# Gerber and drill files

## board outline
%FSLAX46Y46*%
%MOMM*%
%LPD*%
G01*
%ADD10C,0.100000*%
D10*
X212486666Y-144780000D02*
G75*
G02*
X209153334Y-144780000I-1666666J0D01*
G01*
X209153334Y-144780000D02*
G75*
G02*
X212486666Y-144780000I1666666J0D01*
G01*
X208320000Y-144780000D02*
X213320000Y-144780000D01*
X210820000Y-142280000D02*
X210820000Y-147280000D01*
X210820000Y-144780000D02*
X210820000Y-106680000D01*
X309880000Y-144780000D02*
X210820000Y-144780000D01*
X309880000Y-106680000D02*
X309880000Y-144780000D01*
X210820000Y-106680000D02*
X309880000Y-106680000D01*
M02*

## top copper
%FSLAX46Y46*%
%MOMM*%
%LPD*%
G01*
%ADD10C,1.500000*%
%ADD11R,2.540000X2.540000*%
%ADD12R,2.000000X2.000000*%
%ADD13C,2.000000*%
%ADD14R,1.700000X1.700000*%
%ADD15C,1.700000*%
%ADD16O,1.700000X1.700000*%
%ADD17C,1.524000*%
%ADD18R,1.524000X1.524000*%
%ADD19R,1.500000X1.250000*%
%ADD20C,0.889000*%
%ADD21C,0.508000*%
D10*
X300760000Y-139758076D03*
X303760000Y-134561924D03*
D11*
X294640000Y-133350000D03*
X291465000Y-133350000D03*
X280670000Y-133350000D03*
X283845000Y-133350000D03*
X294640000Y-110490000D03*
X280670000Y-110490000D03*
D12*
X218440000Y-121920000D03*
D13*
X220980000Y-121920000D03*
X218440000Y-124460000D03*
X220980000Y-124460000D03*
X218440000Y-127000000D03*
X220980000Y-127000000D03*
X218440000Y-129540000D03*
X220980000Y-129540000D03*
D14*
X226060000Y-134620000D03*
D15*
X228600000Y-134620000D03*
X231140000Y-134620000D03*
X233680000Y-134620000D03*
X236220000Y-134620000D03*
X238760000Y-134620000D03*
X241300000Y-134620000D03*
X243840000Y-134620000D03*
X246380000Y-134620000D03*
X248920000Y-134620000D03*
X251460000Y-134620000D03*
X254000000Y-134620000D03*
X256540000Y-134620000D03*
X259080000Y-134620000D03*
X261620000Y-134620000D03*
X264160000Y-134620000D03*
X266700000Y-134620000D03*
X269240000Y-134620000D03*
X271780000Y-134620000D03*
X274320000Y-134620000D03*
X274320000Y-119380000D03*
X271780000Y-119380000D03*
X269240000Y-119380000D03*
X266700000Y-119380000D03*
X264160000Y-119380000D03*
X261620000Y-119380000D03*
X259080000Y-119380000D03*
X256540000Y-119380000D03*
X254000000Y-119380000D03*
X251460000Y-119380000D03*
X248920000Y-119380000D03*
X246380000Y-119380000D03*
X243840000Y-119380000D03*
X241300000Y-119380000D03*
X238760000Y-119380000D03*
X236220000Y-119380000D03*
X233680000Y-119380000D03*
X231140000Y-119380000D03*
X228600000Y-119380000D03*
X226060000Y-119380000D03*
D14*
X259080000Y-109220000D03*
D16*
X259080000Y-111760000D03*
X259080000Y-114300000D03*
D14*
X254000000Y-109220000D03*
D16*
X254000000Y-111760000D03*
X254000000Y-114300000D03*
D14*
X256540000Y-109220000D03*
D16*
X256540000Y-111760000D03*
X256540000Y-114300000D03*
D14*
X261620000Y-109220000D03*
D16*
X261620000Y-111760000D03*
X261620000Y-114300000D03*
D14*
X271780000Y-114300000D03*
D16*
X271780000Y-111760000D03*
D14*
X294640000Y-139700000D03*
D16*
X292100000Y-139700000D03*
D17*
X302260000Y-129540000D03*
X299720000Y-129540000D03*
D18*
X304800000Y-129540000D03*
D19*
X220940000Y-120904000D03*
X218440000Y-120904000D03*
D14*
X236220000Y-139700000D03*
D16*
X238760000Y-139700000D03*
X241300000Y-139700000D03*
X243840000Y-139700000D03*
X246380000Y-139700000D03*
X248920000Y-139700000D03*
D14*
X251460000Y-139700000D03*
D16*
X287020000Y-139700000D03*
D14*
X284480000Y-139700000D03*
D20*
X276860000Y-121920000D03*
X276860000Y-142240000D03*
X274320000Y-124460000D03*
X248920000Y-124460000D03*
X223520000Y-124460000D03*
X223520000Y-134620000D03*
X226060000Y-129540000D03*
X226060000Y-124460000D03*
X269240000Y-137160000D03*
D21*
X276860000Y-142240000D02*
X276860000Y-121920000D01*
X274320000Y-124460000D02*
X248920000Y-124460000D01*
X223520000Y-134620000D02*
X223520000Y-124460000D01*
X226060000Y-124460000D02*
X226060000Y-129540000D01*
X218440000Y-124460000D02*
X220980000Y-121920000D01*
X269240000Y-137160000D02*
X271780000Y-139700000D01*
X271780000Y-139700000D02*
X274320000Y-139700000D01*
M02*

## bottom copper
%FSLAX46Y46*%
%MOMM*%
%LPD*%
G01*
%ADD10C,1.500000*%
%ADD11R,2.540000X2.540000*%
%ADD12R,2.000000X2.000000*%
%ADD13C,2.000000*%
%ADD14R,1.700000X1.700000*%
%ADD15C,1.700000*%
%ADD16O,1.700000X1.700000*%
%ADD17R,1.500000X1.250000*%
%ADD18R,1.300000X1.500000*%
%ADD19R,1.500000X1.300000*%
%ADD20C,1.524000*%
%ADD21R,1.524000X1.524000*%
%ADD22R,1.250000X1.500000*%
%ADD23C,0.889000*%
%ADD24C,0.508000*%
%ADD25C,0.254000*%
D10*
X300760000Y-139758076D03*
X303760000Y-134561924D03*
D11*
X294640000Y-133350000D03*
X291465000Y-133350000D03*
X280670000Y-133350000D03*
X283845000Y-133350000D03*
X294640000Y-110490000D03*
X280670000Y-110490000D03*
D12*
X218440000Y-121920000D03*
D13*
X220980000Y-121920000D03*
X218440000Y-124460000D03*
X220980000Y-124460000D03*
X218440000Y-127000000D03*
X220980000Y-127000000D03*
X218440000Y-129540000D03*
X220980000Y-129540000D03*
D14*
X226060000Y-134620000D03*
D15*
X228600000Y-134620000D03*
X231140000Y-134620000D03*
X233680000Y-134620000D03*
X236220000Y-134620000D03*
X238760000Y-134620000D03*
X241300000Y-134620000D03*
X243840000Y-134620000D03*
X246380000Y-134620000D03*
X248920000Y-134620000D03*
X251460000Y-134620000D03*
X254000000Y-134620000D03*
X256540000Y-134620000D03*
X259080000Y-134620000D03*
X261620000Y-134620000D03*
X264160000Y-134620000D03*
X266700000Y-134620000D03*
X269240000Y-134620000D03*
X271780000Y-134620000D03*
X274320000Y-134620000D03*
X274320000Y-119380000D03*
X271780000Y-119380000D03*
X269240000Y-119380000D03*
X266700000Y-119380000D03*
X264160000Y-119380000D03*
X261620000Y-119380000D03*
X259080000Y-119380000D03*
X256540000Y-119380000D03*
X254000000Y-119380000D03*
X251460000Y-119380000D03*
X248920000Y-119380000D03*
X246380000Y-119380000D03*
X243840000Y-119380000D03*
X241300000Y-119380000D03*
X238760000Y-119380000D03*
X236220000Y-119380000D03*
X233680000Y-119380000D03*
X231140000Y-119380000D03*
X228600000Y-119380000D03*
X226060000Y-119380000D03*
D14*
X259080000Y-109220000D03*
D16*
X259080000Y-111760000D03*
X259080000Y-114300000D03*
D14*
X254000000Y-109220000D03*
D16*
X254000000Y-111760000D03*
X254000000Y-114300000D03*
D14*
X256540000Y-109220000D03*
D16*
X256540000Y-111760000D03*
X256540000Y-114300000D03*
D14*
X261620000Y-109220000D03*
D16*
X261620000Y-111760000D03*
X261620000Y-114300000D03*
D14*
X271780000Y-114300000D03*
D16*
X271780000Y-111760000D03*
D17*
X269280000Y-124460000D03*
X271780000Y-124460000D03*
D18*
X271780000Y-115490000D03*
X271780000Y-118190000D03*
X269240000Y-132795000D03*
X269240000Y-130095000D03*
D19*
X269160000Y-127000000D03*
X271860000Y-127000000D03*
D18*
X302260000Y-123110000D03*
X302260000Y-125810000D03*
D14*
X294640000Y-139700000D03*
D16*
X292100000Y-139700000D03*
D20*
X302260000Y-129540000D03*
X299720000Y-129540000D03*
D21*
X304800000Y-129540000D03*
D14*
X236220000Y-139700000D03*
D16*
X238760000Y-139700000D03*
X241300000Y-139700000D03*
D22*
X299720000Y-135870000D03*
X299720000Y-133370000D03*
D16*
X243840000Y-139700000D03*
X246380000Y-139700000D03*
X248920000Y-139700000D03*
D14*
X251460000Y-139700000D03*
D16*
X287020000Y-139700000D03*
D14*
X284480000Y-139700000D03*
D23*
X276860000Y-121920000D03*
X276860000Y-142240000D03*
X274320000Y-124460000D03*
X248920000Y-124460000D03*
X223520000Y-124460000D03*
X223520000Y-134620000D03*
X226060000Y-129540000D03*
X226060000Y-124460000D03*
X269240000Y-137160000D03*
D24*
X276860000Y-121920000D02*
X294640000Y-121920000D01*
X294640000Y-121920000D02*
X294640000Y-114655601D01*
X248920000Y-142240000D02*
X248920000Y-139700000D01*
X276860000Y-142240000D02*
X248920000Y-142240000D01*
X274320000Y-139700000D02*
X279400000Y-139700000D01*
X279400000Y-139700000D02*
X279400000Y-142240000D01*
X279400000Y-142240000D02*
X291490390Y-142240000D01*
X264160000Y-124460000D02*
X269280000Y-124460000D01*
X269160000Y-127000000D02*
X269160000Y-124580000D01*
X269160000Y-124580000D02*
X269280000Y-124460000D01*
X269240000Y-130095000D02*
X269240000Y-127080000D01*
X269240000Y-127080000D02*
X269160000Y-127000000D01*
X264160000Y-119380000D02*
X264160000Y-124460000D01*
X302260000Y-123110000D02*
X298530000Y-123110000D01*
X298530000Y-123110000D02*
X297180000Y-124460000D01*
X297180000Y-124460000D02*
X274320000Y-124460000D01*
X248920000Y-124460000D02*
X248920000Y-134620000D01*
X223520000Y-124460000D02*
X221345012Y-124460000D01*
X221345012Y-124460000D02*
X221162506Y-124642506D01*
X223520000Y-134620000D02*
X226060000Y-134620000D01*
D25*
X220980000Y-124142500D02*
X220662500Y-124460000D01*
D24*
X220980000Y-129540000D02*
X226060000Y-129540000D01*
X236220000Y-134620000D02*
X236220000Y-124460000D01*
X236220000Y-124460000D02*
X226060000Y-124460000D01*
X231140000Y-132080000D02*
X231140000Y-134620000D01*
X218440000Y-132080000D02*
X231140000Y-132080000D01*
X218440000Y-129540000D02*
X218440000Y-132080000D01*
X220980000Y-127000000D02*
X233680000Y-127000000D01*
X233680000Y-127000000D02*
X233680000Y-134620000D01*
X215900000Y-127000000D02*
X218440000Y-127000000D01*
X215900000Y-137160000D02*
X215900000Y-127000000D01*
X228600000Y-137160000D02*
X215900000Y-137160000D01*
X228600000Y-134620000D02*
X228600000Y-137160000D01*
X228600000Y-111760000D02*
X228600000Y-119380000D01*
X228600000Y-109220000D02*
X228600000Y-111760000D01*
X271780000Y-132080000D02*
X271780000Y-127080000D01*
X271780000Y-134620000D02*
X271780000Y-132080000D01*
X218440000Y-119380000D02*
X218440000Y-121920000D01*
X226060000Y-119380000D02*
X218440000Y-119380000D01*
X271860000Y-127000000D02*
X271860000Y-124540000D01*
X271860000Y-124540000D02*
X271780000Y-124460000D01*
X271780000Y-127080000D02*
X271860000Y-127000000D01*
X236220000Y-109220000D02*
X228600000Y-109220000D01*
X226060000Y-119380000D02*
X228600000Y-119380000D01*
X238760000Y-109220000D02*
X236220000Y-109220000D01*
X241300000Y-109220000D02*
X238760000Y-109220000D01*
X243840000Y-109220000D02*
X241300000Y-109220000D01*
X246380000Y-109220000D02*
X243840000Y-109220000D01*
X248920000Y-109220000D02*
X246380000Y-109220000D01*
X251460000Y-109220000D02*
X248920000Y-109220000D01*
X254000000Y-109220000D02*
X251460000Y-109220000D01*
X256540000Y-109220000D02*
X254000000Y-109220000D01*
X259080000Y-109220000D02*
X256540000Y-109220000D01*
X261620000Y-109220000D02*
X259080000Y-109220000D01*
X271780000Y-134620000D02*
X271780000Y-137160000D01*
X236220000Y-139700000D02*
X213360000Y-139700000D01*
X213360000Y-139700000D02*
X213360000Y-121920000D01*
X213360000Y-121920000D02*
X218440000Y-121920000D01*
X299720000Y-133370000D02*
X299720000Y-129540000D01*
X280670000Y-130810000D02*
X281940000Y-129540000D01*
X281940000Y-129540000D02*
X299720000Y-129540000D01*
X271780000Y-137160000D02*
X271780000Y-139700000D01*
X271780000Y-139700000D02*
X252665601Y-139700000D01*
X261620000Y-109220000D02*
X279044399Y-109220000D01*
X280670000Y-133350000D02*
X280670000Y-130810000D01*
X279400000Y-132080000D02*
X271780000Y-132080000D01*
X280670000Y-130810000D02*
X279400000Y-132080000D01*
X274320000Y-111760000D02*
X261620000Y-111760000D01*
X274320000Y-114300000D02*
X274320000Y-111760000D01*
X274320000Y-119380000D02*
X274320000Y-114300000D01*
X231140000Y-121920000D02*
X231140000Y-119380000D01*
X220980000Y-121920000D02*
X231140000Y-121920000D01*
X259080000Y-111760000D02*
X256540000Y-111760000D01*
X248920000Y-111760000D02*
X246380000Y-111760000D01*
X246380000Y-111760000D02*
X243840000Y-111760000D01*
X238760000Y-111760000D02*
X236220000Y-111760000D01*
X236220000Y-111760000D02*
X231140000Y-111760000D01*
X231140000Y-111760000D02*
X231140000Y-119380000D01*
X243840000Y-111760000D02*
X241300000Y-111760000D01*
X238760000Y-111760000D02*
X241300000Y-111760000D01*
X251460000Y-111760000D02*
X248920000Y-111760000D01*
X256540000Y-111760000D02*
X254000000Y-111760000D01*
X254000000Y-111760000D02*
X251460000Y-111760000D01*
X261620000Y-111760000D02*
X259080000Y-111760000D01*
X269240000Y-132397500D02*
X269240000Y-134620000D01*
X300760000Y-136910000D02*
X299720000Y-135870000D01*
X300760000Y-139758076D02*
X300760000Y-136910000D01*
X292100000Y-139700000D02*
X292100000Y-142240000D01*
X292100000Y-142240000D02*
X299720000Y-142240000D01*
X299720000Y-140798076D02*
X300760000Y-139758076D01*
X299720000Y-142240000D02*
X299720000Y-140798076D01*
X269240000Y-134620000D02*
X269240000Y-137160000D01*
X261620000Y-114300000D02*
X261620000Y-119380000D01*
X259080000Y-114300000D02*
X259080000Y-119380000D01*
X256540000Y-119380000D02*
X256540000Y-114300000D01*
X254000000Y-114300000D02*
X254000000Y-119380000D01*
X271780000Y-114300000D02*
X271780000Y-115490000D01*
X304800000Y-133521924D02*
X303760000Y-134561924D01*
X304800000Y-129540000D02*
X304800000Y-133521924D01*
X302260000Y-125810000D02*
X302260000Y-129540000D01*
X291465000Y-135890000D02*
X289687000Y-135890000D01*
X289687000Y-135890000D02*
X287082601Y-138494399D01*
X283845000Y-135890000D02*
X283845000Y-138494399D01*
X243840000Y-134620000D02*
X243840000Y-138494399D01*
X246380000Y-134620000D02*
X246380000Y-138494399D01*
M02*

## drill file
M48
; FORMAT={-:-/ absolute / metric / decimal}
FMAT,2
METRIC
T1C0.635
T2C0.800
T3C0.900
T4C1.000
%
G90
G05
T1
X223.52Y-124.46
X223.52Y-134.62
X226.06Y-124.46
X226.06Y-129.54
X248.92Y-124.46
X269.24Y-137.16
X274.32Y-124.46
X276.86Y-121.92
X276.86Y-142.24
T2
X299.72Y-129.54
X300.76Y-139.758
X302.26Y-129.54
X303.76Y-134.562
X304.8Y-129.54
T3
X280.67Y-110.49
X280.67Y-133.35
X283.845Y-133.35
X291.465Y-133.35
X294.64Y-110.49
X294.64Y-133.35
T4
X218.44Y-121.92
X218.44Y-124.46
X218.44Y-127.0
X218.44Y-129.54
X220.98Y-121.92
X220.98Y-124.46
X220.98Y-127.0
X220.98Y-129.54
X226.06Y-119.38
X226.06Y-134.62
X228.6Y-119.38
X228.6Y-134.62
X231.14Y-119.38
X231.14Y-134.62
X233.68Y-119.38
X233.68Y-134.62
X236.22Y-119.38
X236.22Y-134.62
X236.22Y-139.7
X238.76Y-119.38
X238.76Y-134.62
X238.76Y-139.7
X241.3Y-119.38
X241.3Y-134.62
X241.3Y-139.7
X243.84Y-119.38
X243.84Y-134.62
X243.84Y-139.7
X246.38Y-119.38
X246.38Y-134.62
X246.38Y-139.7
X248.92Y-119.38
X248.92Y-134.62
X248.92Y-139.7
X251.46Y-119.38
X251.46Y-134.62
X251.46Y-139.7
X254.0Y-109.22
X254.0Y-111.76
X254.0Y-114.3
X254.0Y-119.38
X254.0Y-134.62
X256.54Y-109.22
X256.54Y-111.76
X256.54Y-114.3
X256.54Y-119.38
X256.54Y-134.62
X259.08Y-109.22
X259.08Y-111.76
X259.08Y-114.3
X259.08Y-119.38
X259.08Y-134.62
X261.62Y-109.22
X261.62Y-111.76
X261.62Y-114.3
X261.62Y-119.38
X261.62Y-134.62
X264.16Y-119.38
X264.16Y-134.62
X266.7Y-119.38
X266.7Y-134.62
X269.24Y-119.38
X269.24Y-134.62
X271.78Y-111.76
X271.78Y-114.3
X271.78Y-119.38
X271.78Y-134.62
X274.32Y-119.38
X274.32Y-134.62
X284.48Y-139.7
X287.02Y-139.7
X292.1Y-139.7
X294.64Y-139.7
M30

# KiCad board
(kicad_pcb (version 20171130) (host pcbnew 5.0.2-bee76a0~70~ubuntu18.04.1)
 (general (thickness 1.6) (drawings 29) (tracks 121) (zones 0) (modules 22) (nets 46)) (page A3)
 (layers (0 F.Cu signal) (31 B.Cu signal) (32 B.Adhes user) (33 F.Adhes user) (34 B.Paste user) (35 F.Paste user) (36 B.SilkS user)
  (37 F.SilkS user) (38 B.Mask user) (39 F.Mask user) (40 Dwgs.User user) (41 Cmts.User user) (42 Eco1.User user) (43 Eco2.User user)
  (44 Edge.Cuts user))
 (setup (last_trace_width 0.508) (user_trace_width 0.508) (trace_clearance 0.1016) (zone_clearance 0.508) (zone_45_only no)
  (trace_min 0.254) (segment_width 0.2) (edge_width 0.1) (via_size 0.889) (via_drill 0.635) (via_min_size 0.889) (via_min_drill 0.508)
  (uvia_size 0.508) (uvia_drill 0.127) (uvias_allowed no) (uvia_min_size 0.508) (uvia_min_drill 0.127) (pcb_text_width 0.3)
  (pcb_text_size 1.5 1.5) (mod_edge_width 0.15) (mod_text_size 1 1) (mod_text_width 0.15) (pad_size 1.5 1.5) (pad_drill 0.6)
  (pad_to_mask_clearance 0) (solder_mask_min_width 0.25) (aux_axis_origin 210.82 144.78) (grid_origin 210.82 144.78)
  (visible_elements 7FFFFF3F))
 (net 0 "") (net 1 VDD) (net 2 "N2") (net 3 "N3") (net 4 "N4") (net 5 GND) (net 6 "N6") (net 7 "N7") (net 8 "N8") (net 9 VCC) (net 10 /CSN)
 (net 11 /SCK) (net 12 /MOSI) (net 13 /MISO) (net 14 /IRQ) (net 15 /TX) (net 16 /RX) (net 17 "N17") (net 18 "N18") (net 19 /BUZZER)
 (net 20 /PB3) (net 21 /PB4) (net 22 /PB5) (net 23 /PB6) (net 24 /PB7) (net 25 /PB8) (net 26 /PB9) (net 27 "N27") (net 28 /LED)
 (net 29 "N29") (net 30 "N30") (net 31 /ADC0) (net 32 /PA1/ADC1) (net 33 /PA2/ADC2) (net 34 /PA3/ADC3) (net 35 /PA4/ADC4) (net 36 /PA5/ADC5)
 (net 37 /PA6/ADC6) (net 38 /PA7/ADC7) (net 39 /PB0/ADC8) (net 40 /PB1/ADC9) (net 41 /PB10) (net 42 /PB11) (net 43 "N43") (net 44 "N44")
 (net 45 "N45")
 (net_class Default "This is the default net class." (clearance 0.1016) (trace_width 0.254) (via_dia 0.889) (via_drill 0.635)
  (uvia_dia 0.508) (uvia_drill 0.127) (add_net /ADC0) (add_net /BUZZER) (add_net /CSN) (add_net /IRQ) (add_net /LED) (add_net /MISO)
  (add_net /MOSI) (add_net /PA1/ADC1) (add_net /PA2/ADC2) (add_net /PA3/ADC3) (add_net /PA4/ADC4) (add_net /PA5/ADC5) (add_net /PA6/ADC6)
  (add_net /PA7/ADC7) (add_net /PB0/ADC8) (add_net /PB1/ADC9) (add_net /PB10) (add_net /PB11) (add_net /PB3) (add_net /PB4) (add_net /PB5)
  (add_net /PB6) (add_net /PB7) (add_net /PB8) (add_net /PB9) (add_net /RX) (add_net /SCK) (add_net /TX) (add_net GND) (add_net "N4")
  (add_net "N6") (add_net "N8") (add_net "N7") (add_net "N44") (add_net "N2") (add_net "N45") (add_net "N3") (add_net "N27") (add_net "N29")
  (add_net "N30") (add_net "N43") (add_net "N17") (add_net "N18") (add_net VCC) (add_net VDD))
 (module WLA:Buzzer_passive (layer F.Cu) (at 302.26 137.16 60)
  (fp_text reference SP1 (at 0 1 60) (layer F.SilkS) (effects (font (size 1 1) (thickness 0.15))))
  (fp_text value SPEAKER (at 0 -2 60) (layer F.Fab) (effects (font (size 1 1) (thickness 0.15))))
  (pad 1 thru_hole circle (at -3 0 60) (size 1.5 1.5) (drill 0.8) (layers *.Cu *.Mask) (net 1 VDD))
  (pad 2 thru_hole circle (at 3 0 60) (size 1.5 1.5) (drill 0.8) (layers *.Cu *.Mask) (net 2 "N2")))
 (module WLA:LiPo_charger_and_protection (layer F.Cu) (at 287.655 121.92 270)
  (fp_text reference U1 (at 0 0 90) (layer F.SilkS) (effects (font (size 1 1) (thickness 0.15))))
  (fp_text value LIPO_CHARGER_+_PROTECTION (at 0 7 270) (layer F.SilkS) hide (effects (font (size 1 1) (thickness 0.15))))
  (pad 3 thru_hole rect (at 11.43 -6.985 270) (size 2.54 2.54) (drill 0.9) (layers *.Cu *.Mask F.SilkS) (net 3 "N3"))
  (pad 1 thru_hole rect (at 11.43 -3.81 270) (size 2.54 2.54) (drill 0.9) (layers *.Cu *.Mask F.SilkS) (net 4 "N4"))
  (pad 4 thru_hole rect (at 11.43 6.985 270) (size 2.54 2.54) (drill 0.9) (layers *.Cu *.Mask F.SilkS) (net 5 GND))
  (pad 2 thru_hole rect (at 11.43 3.81 270) (size 2.54 2.54) (drill 0.9) (layers *.Cu *.Mask F.SilkS) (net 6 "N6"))
  (pad 5 thru_hole rect (at -11.43 -6.985 270) (size 2.54 2.54) (drill 0.9) (layers *.Cu *.Mask F.SilkS) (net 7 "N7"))
  (pad 6 thru_hole rect (at -11.43 6.985 270) (size 2.54 2.54) (drill 0.9) (layers *.Cu *.Mask F.SilkS) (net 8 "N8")))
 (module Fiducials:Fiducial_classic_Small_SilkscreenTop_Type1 (layer F.Cu) (at 210.82 144.78)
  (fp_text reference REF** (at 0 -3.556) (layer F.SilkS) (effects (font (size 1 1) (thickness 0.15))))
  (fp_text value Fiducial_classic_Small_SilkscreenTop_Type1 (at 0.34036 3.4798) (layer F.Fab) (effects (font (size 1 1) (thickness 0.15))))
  (pad ~ smd circle (at 0 0) (size 4.50088 4.50088) (layers F.Mask) (solder_mask_margin 2.99974)))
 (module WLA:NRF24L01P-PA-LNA (layer F.Cu) (at 218.44 125.73 270)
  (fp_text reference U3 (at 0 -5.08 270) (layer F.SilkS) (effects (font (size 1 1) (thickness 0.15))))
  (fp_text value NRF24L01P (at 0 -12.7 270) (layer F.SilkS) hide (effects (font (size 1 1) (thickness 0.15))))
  (pad 1 thru_hole rect (at -3.81 0 270) (size 2 2) (drill 1) (layers *.Cu *.Mask F.SilkS) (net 5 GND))
  (pad 2 thru_hole circle (at -3.81 -2.54 270) (size 2 2) (drill 1) (layers *.Cu *.Mask F.SilkS) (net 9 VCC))
  (pad 3 thru_hole circle (at -1.27 0 270) (size 2 2) (drill 1) (layers *.Cu *.Mask F.SilkS) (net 9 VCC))
  (pad 4 thru_hole circle (at -1.27 -2.54 270) (size 2 2) (drill 1) (layers *.Cu *.Mask F.SilkS) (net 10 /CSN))
  (pad 5 thru_hole circle (at 1.27 0 270) (size 2 2) (drill 1) (layers *.Cu *.Mask F.SilkS) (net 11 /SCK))
  (pad 6 thru_hole circle (at 1.27 -2.54 270) (size 2 2) (drill 1) (layers *.Cu *.Mask F.SilkS) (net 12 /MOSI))
  (pad 7 thru_hole circle (at 3.81 0 270) (size 2 2) (drill 1) (layers *.Cu *.Mask F.SilkS) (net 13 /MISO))
  (pad 8 thru_hole circle (at 3.81 -2.54 270) (size 2 2) (drill 1) (layers *.Cu *.Mask F.SilkS) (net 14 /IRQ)))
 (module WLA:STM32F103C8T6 (layer F.Cu) (at 250.19 127)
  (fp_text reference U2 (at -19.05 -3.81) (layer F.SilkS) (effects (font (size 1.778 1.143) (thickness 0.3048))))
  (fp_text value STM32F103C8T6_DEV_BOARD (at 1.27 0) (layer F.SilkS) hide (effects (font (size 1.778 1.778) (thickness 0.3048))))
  (pad 1 thru_hole rect (at -24.13 7.62) (size 1.7 1.7) (drill 1) (layers *.Cu *.Mask F.SilkS) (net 10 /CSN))
  (pad 2 thru_hole circle (at -21.59 7.62) (size 1.7 1.7) (drill 1) (layers *.Cu *.Mask F.SilkS) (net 11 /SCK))
  (pad 3 thru_hole circle (at -19.05 7.62) (size 1.7 1.7) (drill 1) (layers *.Cu *.Mask F.SilkS) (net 13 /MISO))
  (pad 4 thru_hole circle (at -16.51 7.62) (size 1.7 1.7) (drill 1) (layers *.Cu *.Mask F.SilkS) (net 12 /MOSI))
  (pad 5 thru_hole circle (at -13.97 7.62) (size 1.7 1.7) (drill 1) (layers *.Cu *.Mask F.SilkS) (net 14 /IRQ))
  (pad 6 thru_hole circle (at -11.43 7.62) (size 1.7 1.7) (drill 1) (layers *.Cu *.Mask F.SilkS) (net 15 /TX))
  (pad 7 thru_hole circle (at -8.89 7.62) (size 1.7 1.7) (drill 1) (layers *.Cu *.Mask F.SilkS) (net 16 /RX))
  (pad 8 thru_hole circle (at -6.35 7.62) (size 1.7 1.7) (drill 1) (layers *.Cu *.Mask F.SilkS) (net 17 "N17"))
  (pad 9 thru_hole circle (at -3.81 7.62) (size 1.7 1.7) (drill 1) (layers *.Cu *.Mask F.SilkS) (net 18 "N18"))
  (pad 10 thru_hole circle (at -1.27 7.62) (size 1.7 1.7) (drill 1) (layers *.Cu *.Mask F.SilkS) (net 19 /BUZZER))
  (pad 11 thru_hole circle (at 1.27 7.62) (size 1.7 1.7) (drill 1) (layers *.Cu *.Mask F.SilkS) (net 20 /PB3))
  (pad 12 thru_hole circle (at 3.81 7.62) (size 1.7 1.7) (drill 1) (layers *.Cu *.Mask F.SilkS) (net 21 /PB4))
  (pad 13 thru_hole circle (at 6.35 7.62) (size 1.7 1.7) (drill 1) (layers *.Cu *.Mask F.SilkS) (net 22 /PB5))
  (pad 14 thru_hole circle (at 8.89 7.62) (size 1.7 1.7) (drill 1) (layers *.Cu *.Mask F.SilkS) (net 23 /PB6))
  (pad 15 thru_hole circle (at 11.43 7.62) (size 1.7 1.7) (drill 1) (layers *.Cu *.Mask F.SilkS) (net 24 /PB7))
  (pad 16 thru_hole circle (at 13.97 7.62) (size 1.7 1.7) (drill 1) (layers *.Cu *.Mask F.SilkS) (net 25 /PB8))
  (pad 17 thru_hole circle (at 16.51 7.62) (size 1.7 1.7) (drill 1) (layers *.Cu *.Mask F.SilkS) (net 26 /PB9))
  (pad 18 thru_hole circle (at 19.05 7.62) (size 1.7 1.7) (drill 1) (layers *.Cu *.Mask F.SilkS) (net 1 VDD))
  (pad 19 thru_hole circle (at 21.59 7.62) (size 1.7 1.7) (drill 1) (layers *.Cu *.Mask F.SilkS) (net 5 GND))
  (pad 20 thru_hole circle (at 24.13 7.62) (size 1.7 1.7) (drill 1) (layers *.Cu *.Mask F.SilkS) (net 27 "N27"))
  (pad 21 thru_hole circle (at 24.13 -7.62) (size 1.7 1.7) (drill 1) (layers *.Cu *.Mask F.SilkS) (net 9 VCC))
  (pad 22 thru_hole circle (at 21.59 -7.62) (size 1.7 1.7) (drill 1) (layers *.Cu *.Mask F.SilkS) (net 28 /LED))
  (pad 23 thru_hole circle (at 19.05 -7.62) (size 1.7 1.7) (drill 1) (layers *.Cu *.Mask F.SilkS) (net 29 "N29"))
  (pad 24 thru_hole circle (at 16.51 -7.62) (size 1.7 1.7) (drill 1) (layers *.Cu *.Mask F.SilkS) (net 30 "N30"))
  (pad 25 thru_hole circle (at 13.97 -7.62) (size 1.7 1.7) (drill 1) (layers *.Cu *.Mask F.SilkS) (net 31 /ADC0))
  (pad 26 thru_hole circle (at 11.43 -7.62) (size 1.7 1.7) (drill 1) (layers *.Cu *.Mask F.SilkS) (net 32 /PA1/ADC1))
  (pad 27 thru_hole circle (at 8.89 -7.62) (size 1.7 1.7) (drill 1) (layers *.Cu *.Mask F.SilkS) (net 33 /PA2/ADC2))
  (pad 28 thru_hole circle (at 6.35 -7.62) (size 1.7 1.7) (drill 1) (layers *.Cu *.Mask F.SilkS) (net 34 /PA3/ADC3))
  (pad 29 thru_hole circle (at 3.81 -7.62) (size 1.7 1.7) (drill 1) (layers *.Cu *.Mask F.SilkS) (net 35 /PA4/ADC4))
  (pad 30 thru_hole circle (at 1.27 -7.62) (size 1.7 1.7) (drill 1) (layers *.Cu *.Mask F.SilkS) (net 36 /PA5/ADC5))
  (pad 31 thru_hole circle (at -1.27 -7.62) (size 1.7 1.7) (drill 1) (layers *.Cu *.Mask F.SilkS) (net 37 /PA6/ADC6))
  (pad 32 thru_hole circle (at -3.81 -7.62) (size 1.7 1.7) (drill 1) (layers *.Cu *.Mask F.SilkS) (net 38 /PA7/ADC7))
  (pad 33 thru_hole circle (at -6.35 -7.62) (size 1.7 1.7) (drill 1) (layers *.Cu *.Mask F.SilkS) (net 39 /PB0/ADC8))
  (pad 34 thru_hole circle (at -8.89 -7.62) (size 1.7 1.7) (drill 1) (layers *.Cu *.Mask F.SilkS) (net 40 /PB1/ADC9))
  (pad 35 thru_hole circle (at -11.43 -7.62) (size 1.7 1.7) (drill 1) (layers *.Cu *.Mask F.SilkS) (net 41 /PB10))
  (pad 36 thru_hole circle (at -13.97 -7.62) (size 1.7 1.7) (drill 1) (layers *.Cu *.Mask F.SilkS) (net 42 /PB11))
  (pad 37 thru_hole circle (at -16.51 -7.62) (size 1.7 1.7) (drill 1) (layers *.Cu *.Mask F.SilkS) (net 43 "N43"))
  (pad 38 thru_hole circle (at -19.05 -7.62) (size 1.7 1.7) (drill 1) (layers *.Cu *.Mask F.SilkS) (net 9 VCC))
  (pad 39 thru_hole circle (at -21.59 -7.62) (size 1.7 1.7) (drill 1) (layers *.Cu *.Mask F.SilkS) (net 5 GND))
  (pad 40 thru_hole circle (at -24.13 -7.62) (size 1.7 1.7) (drill 1) (layers *.Cu *.Mask F.SilkS) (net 5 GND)))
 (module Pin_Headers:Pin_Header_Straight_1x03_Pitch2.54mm (layer F.Cu) (at 259.08 109.22)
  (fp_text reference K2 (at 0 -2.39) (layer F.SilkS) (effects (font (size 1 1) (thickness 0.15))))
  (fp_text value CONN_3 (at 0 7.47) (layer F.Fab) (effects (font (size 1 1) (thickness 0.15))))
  (pad 1 thru_hole rect (at 0 0) (size 1.7 1.7) (drill 1) (layers *.Cu *.Mask) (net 5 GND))
  (pad 2 thru_hole oval (at 0 2.54) (size 1.7 1.7) (drill 1) (layers *.Cu *.Mask) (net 9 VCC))
  (pad 3 thru_hole oval (at 0 5.08) (size 1.7 1.7) (drill 1) (layers *.Cu *.Mask) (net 33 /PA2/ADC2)))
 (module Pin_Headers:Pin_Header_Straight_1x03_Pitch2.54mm (layer F.Cu) (at 254 109.22)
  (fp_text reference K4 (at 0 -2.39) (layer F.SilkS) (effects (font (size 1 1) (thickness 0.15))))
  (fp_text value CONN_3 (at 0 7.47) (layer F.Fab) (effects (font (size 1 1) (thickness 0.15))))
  (pad 1 thru_hole rect (at 0 0) (size 1.7 1.7) (drill 1) (layers *.Cu *.Mask) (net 5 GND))
  (pad 2 thru_hole oval (at 0 2.54) (size 1.7 1.7) (drill 1) (layers *.Cu *.Mask) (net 9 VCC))
  (pad 3 thru_hole oval (at 0 5.08) (size 1.7 1.7) (drill 1) (layers *.Cu *.Mask) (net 35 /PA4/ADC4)))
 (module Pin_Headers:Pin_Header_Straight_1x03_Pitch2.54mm (layer F.Cu) (at 256.54 109.22)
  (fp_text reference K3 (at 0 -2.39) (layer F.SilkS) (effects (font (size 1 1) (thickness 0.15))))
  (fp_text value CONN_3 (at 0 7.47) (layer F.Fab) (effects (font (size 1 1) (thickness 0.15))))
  (pad 1 thru_hole rect (at 0 0) (size 1.7 1.7) (drill 1) (layers *.Cu *.Mask) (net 5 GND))
  (pad 2 thru_hole oval (at 0 2.54) (size 1.7 1.7) (drill 1) (layers *.Cu *.Mask) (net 9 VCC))
  (pad 3 thru_hole oval (at 0 5.08) (size 1.7 1.7) (drill 1) (layers *.Cu *.Mask) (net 34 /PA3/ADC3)))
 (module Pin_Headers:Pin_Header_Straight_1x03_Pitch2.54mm (layer F.Cu) (at 261.62 109.22)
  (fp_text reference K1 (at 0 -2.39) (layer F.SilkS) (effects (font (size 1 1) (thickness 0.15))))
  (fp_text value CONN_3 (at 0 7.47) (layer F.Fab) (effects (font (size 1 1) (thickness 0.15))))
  (pad 1 thru_hole rect (at 0 0) (size 1.7 1.7) (drill 1) (layers *.Cu *.Mask) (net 5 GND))
  (pad 2 thru_hole oval (at 0 2.54) (size 1.7 1.7) (drill 1) (layers *.Cu *.Mask) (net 9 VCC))
  (pad 3 thru_hole oval (at 0 5.08) (size 1.7 1.7) (drill 1) (layers *.Cu *.Mask) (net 32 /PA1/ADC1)))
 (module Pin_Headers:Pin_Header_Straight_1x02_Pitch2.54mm (layer F.Cu) (at 271.78 114.3 180)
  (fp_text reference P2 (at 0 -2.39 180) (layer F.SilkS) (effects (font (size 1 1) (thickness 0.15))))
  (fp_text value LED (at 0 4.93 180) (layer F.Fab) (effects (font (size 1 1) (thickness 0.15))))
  (pad 1 thru_hole rect (at 0 0 180) (size 1.7 1.7) (drill 1) (layers *.Cu *.Mask) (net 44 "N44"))
  (pad 2 thru_hole oval (at 0 2.54 180) (size 1.7 1.7) (drill 1) (layers *.Cu *.Mask) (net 9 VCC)))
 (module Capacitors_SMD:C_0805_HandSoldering (layer B.Cu) (at 270.53 124.46)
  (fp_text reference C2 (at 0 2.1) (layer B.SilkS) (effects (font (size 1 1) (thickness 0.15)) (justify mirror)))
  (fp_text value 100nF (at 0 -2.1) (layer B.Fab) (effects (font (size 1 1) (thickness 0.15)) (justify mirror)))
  (pad 1 smd rect (at -1.25 0) (size 1.5 1.25) (layers B.Cu B.Paste B.Mask) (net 31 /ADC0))
  (pad 2 smd rect (at 1.25 0) (size 1.5 1.25) (layers B.Cu B.Paste B.Mask) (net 5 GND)))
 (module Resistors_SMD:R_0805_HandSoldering (layer B.Cu) (at 271.78 116.84 270)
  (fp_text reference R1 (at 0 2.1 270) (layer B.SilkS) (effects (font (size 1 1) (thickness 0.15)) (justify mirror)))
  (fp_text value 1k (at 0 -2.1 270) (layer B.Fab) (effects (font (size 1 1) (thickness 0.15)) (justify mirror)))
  (pad 1 smd rect (at -1.35 0 270) (size 1.5 1.3) (layers B.Cu B.Paste B.Mask) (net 44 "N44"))
  (pad 2 smd rect (at 1.35 0 270) (size 1.5 1.3) (layers B.Cu B.Paste B.Mask) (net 28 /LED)))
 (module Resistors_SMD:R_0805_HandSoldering (layer B.Cu) (at 269.24 131.445 90)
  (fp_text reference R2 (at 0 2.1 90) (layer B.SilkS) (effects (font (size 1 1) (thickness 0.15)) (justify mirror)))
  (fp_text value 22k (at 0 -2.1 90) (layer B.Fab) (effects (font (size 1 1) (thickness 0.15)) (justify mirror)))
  (pad 1 smd rect (at -1.35 0 90) (size 1.5 1.3) (layers B.Cu B.Paste B.Mask) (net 1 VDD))
  (pad 2 smd rect (at 1.35 0 90) (size 1.5 1.3) (layers B.Cu B.Paste B.Mask) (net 31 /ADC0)))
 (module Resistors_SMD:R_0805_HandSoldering (layer B.Cu) (at 270.51 127)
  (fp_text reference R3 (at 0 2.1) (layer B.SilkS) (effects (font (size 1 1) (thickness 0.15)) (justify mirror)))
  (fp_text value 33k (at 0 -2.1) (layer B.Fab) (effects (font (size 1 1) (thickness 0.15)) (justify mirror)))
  (pad 1 smd rect (at -1.35 0) (size 1.5 1.3) (layers B.Cu B.Paste B.Mask) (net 31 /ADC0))
  (pad 2 smd rect (at 1.35 0) (size 1.5 1.3) (layers B.Cu B.Paste B.Mask) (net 5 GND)))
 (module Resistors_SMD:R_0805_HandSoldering (layer B.Cu) (at 302.26 124.46 270)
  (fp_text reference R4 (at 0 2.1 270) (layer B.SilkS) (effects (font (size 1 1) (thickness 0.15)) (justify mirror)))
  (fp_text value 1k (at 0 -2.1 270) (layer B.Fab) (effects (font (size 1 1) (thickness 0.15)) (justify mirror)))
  (pad 1 smd rect (at -1.35 0 270) (size 1.5 1.3) (layers B.Cu B.Paste B.Mask) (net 19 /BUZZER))
  (pad 2 smd rect (at 1.35 0 270) (size 1.5 1.3) (layers B.Cu B.Paste B.Mask) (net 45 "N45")))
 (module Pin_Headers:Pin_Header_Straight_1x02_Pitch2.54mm (layer F.Cu) (at 294.64 139.7 270)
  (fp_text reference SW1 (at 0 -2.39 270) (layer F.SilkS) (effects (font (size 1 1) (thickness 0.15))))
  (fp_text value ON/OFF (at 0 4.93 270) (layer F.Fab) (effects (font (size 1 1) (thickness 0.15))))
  (pad 1 thru_hole rect (at 0 0 270) (size 1.7 1.7) (drill 1) (layers *.Cu *.Mask) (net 3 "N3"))
  (pad 2 thru_hole oval (at 0 2.54 270) (size 1.7 1.7) (drill 1) (layers *.Cu *.Mask) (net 1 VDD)))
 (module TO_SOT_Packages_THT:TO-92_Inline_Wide (layer F.Cu) (at 304.8 129.54 180)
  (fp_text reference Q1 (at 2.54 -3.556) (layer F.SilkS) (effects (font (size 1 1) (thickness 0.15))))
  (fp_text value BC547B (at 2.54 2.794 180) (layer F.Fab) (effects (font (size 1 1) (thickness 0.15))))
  (pad 2 thru_hole circle (at 2.54 0 270) (size 1.524 1.524) (drill 0.8) (layers *.Cu *.Mask) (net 45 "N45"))
  (pad 3 thru_hole circle (at 5.08 0 270) (size 1.524 1.524) (drill 0.8) (layers *.Cu *.Mask) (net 5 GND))
  (pad 1 thru_hole rect (at 0 0 270) (size 1.524 1.524) (drill 0.8) (layers *.Cu *.Mask) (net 2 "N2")))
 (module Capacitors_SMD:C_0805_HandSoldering (layer F.Cu) (at 219.69 120.904 180)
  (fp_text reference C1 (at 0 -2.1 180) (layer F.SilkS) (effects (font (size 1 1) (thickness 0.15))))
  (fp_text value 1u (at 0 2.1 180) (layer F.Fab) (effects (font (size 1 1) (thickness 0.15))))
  (pad 1 smd rect (at -1.25 0 180) (size 1.5 1.25) (layers F.Cu F.Paste F.Mask) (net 9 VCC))
  (pad 2 smd rect (at 1.25 0 180) (size 1.5 1.25) (layers F.Cu F.Paste F.Mask) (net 5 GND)))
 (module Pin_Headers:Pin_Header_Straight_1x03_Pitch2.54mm (layer F.Cu) (at 236.22 139.7 90)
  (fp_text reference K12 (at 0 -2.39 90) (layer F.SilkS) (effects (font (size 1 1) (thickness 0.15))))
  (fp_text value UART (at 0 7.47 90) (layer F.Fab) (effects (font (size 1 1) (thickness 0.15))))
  (pad 1 thru_hole rect (at 0 0 90) (size 1.7 1.7) (drill 1) (layers *.Cu *.Mask) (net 5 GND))
  (pad 2 thru_hole oval (at 0 2.54 90) (size 1.7 1.7) (drill 1) (layers *.Cu *.Mask) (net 16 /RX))
  (pad 3 thru_hole oval (at 0 5.08 90) (size 1.7 1.7) (drill 1) (layers *.Cu *.Mask) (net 15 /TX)))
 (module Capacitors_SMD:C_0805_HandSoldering (layer B.Cu) (at 299.72 134.62 90)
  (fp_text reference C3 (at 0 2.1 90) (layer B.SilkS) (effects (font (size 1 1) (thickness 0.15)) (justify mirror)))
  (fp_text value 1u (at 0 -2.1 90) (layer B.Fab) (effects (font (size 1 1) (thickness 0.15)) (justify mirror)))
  (pad 1 smd rect (at -1.25 0 90) (size 1.5 1.25) (layers B.Cu B.Paste B.Mask) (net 1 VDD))
  (pad 2 smd rect (at 1.25 0 90) (size 1.5 1.25) (layers B.Cu B.Paste B.Mask) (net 5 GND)))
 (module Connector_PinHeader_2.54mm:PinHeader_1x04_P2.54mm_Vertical (layer F.Cu) (at 251.46 139.7 270)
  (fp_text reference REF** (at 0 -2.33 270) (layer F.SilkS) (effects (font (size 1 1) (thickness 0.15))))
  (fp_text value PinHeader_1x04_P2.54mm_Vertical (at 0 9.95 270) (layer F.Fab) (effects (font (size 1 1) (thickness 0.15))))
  (pad 4 thru_hole oval (at 0 7.62 270) (size 1.7 1.7) (drill 1) (layers *.Cu *.Mask))
  (pad 3 thru_hole oval (at 0 5.08 270) (size 1.7 1.7) (drill 1) (layers *.Cu *.Mask))
  (pad 2 thru_hole oval (at 0 2.54 270) (size 1.7 1.7) (drill 1) (layers *.Cu *.Mask))
  (pad 1 thru_hole rect (at 0 0 270) (size 1.7 1.7) (drill 1) (layers *.Cu *.Mask)))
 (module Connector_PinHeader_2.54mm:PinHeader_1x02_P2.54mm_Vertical (layer F.Cu) (at 284.48 139.7 90)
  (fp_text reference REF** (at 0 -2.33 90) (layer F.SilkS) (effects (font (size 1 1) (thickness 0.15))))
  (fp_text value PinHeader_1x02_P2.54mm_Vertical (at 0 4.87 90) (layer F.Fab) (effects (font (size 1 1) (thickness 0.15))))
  (pad 2 thru_hole oval (at 0 2.54 90) (size 1.7 1.7) (drill 1) (layers *.Cu *.Mask))
  (pad 1 thru_hole rect (at 0 0 90) (size 1.7 1.7) (drill 1) (layers *.Cu *.Mask)))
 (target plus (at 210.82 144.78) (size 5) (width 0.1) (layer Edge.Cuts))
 (gr_line (start 210.82 144.78) (end 210.82 106.68) (layer Edge.Cuts) (width 0.1))
 (gr_line (start 309.88 144.78) (end 210.82 144.78) (layer Edge.Cuts) (width 0.1))
 (gr_line (start 309.88 106.68) (end 309.88 144.78) (layer Edge.Cuts) (width 0.1))
 (gr_line (start 210.82 106.68) (end 309.88 106.68) (layer Edge.Cuts) (width 0.1))
 (via (at 276.86 121.92) (size 0.889) (drill 0.635) (layers F.Cu B.Cu) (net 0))
 (segment (start 276.86 121.92) (end 294.64 121.92) (width 0.508) (layer B.Cu) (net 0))
 (segment (start 294.64 121.92) (end 294.64 114.655601) (width 0.508) (layer B.Cu) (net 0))
 (via (at 276.86 142.24) (size 0.889) (drill 0.635) (layers F.Cu B.Cu) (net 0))
 (segment (start 276.86 142.24) (end 276.86 121.92) (width 0.508) (layer F.Cu) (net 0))
 (segment (start 248.92 142.24) (end 248.92 139.7) (width 0.508) (layer B.Cu) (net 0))
 (segment (start 276.86 142.24) (end 248.92 142.24) (width 0.508) (layer B.Cu) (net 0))
 (segment (start 274.32 139.7) (end 279.4 139.7) (width 0.508) (layer B.Cu) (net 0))
 (segment (start 279.4 139.7) (end 279.4 142.24) (width 0.508) (layer B.Cu) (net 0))
 (segment (start 279.4 142.24) (end 291.49039 142.24) (width 0.508) (layer B.Cu) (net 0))
 (segment (start 264.16 124.46) (end 269.28 124.46) (width 0.508) (layer B.Cu) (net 31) (status 20))
 (segment (start 269.16 127) (end 269.16 124.58) (width 0.508) (layer B.Cu) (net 31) (status 30))
 (segment (start 269.16 124.58) (end 269.28 124.46) (width 0.508) (layer B.Cu) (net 31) (status 30))
 (segment (start 269.24 130.095) (end 269.24 127.08) (width 0.508) (layer B.Cu) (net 31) (status 30))
 (segment (start 269.24 127.08) (end 269.16 127) (width 0.508) (layer B.Cu) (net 31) (status 30))
 (segment (start 264.16 119.38) (end 264.16 124.46) (width 0.508) (layer B.Cu) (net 31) (status 10))
 (segment (start 302.26 123.11) (end 298.53 123.11) (width 0.508) (layer B.Cu) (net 19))
 (segment (start 298.53 123.11) (end 297.18 124.46) (width 0.508) (layer B.Cu) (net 19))
 (segment (start 297.18 124.46) (end 274.32 124.46) (width 0.508) (layer B.Cu) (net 19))
 (via (at 274.32 124.46) (size 0.889) (drill 0.635) (layers F.Cu B.Cu) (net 19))
 (segment (start 274.32 124.46) (end 248.92 124.46) (width 0.508) (layer F.Cu) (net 19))
 (via (at 248.92 124.46) (size 0.889) (drill 0.635) (layers F.Cu B.Cu) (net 19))
 (segment (start 248.92 124.46) (end 248.92 134.62) (width 0.508) (layer B.Cu) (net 19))
 (segment (start 223.52 124.46) (end 221.345012 124.46) (width 0.508) (layer B.Cu) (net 10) (status 20))
 (segment (start 221.345012 124.46) (end 221.162506 124.642506) (width 0.508) (layer B.Cu) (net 10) (status 30))
 (segment (start 223.52 134.62) (end 223.52 124.46) (width 0.508) (layer F.Cu) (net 10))
 (via (at 223.52 124.46) (size 0.889) (drill 0.635) (layers F.Cu B.Cu) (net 10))
 (segment (start 223.52 134.62) (end 226.06 134.62) (width 0.508) (layer B.Cu) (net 10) (status 20))
 (via (at 223.52 134.62) (size 0.889) (drill 0.635) (layers F.Cu B.Cu) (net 10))
 (segment (start 220.98 124.1425) (end 220.6625 124.46) (width 0.254) (layer B.Cu) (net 10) (status 30))
 (segment (start 220.98 129.54) (end 226.06 129.54) (width 0.508) (layer B.Cu) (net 14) (status 10))
 (segment (start 226.06 124.46) (end 226.06 129.54) (width 0.508) (layer F.Cu) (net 14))
 (via (at 226.06 129.54) (size 0.889) (drill 0.635) (layers F.Cu B.Cu) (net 14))
 (segment (start 236.22 134.62) (end 236.22 124.46) (width 0.508) (layer B.Cu) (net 14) (status 10))
 (segment (start 236.22 124.46) (end 226.06 124.46) (width 0.508) (layer B.Cu) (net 14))
 (via (at 226.06 124.46) (size 0.889) (drill 0.635) (layers F.Cu B.Cu) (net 14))
 (segment (start 231.14 132.08) (end 231.14 134.62) (width 0.508) (layer B.Cu) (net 13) (status 20))
 (segment (start 218.44 132.08) (end 231.14 132.08) (width 0.508) (layer B.Cu) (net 13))
 (segment (start 218.44 129.54) (end 218.44 132.08) (width 0.508) (layer B.Cu) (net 13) (status 10))
 (segment (start 220.98 127) (end 233.68 127) (width 0.508) (layer B.Cu) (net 12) (status 10))
 (segment (start 233.68 127) (end 233.68 134.62) (width 0.508) (layer B.Cu) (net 12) (status 20))
 (segment (start 215.9 127) (end 218.44 127) (width 0.508) (layer B.Cu) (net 11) (status 20))
 (segment (start 215.9 137.16) (end 215.9 127) (width 0.508) (layer B.Cu) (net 11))
 (segment (start 228.6 137.16) (end 215.9 137.16) (width 0.508) (layer B.Cu) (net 11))
 (segment (start 228.6 134.62) (end 228.6 137.16) (width 0.508) (layer B.Cu) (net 11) (status 10))
 (segment (start 228.6 111.76) (end 228.6 119.38) (width 0.508) (layer B.Cu) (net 5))
 (segment (start 228.6 109.22) (end 228.6 111.76) (width 0.508) (layer B.Cu) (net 5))
 (segment (start 271.78 132.08) (end 271.78 127.08) (width 0.508) (layer B.Cu) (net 5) (status 20))
 (segment (start 271.78 134.62) (end 271.78 132.08) (width 0.508) (layer B.Cu) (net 5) (status 10))
 (segment (start 218.44 119.38) (end 218.44 121.92) (width 0.508) (layer B.Cu) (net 5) (status 20))
 (segment (start 226.06 119.38) (end 218.44 119.38) (width 0.508) (layer B.Cu) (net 5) (status 10))
 (segment (start 271.86 127) (end 271.86 124.54) (width 0.508) (layer B.Cu) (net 5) (status 30))
 (segment (start 271.86 124.54) (end 271.78 124.46) (width 0.508) (layer B.Cu) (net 5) (status 30))
 (segment (start 271.78 127.08) (end 271.86 127) (width 0.508) (layer B.Cu) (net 5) (status 30))
 (segment (start 236.22 109.22) (end 228.6 109.22) (width 0.508) (layer B.Cu) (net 5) (status 10))
 (segment (start 226.06 119.38) (end 228.6 119.38) (width 0.508) (layer B.Cu) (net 5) (status 30))
 (segment (start 238.76 109.22) (end 236.22 109.22) (width 0.508) (layer B.Cu) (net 5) (status 30))
 (segment (start 241.3 109.22) (end 238.76 109.22) (width 0.508) (layer B.Cu) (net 5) (status 30))
 (segment (start 243.84 109.22) (end 241.3 109.22) (width 0.508) (layer B.Cu) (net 5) (status 30))
 (segment (start 246.38 109.22) (end 243.84 109.22) (width 0.508) (layer B.Cu) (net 5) (status 30))
 (segment (start 248.92 109.22) (end 246.38 109.22) (width 0.508) (layer B.Cu) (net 5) (status 30))
 (segment (start 251.46 109.22) (end 248.92 109.22) (width 0.508) (layer B.Cu) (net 5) (status 30))
 (segment (start 254 109.22) (end 251.46 109.22) (width 0.508) (layer B.Cu) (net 5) (status 30))
 (segment (start 256.54 109.22) (end 254 109.22) (width 0.508) (layer B.Cu) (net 5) (status 30))
 (segment (start 259.08 109.22) (end 256.54 109.22) (width 0.508) (layer B.Cu) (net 5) (status 30))
 (segment (start 261.62 109.22) (end 259.08 109.22) (width 0.508) (layer B.Cu) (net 5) (status 30))
 (segment (start 271.78 134.62) (end 271.78 137.16) (width 0.508) (layer B.Cu) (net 5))
 (segment (start 236.22 139.7) (end 213.36 139.7) (width 0.508) (layer B.Cu) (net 5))
 (segment (start 213.36 139.7) (end 213.36 121.92) (width 0.508) (layer B.Cu) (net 5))
 (segment (start 213.36 121.92) (end 218.44 121.92) (width 0.508) (layer B.Cu) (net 5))
 (segment (start 299.72 133.37) (end 299.72 129.54) (width 0.508) (layer B.Cu) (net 5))
 (segment (start 280.67 130.81) (end 281.94 129.54) (width 0.508) (layer B.Cu) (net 5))
 (segment (start 281.94 129.54) (end 299.72 129.54) (width 0.508) (layer B.Cu) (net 5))
 (segment (start 271.78 137.16) (end 271.78 139.7) (width 0.508) (layer B.Cu) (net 5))
 (segment (start 271.78 139.7) (end 252.665601 139.7) (width 0.508) (layer B.Cu) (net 5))
 (segment (start 261.62 109.22) (end 279.044399 109.22) (width 0.508) (layer B.Cu) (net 5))
 (segment (start 280.67 133.35) (end 280.67 130.81) (width 0.508) (layer B.Cu) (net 5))
 (segment (start 279.4 132.08) (end 271.78 132.08) (width 0.508) (layer B.Cu) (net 5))
 (segment (start 280.67 130.81) (end 279.4 132.08) (width 0.508) (layer B.Cu) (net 5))
 (segment (start 274.32 111.76) (end 261.62 111.76) (width 0.508) (layer B.Cu) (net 9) (status 20))
 (segment (start 274.32 114.3) (end 274.32 111.76) (width 0.508) (layer B.Cu) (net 9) (status 10))
 (segment (start 274.32 119.38) (end 274.32 114.3) (width 0.508) (layer B.Cu) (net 9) (status 30))
 (segment (start 218.44 124.46) (end 220.98 121.92) (width 0.508) (layer F.Cu) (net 9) (status 30))
 (segment (start 231.14 121.92) (end 231.14 119.38) (width 0.508) (layer B.Cu) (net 9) (status 20))
 (segment (start 220.98 121.92) (end 231.14 121.92) (width 0.508) (layer B.Cu) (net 9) (status 10))
 (segment (start 259.08 111.76) (end 256.54 111.76) (width 0.508) (layer B.Cu) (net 9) (status 30))
 (segment (start 248.92 111.76) (end 246.38 111.76) (width 0.508) (layer B.Cu) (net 9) (status 30))
 (segment (start 246.38 111.76) (end 243.84 111.76) (width 0.508) (layer B.Cu) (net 9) (status 30))
 (segment (start 238.76 111.76) (end 236.22 111.76) (width 0.508) (layer B.Cu) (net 9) (status 30))
 (segment (start 236.22 111.76) (end 231.14 111.76) (width 0.508) (layer B.Cu) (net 9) (status 10))
 (segment (start 231.14 111.76) (end 231.14 119.38) (width 0.508) (layer B.Cu) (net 9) (status 20))
 (segment (start 243.84 111.76) (end 241.3 111.76) (width 0.508) (layer B.Cu) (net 9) (status 30))
 (segment (start 238.76 111.76) (end 241.3 111.76) (width 0.508) (layer B.Cu) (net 9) (status 30))
 (segment (start 251.46 111.76) (end 248.92 111.76) (width 0.508) (layer B.Cu) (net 9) (status 30))
 (segment (start 256.54 111.76) (end 254 111.76) (width 0.508) (layer B.Cu) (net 9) (status 30))
 (segment (start 254 111.76) (end 251.46 111.76) (width 0.508) (layer B.Cu) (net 9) (status 30))
 (segment (start 261.62 111.76) (end 259.08 111.76) (width 0.508) (layer B.Cu) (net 9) (status 30))
 (segment (start 269.24 132.3975) (end 269.24 134.62) (width 0.508) (layer B.Cu) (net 1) (status 30))
 (segment (start 300.76 136.91) (end 299.72 135.87) (width 0.508) (layer B.Cu) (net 1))
 (segment (start 300.76 139.758076) (end 300.76 136.91) (width 0.508) (layer B.Cu) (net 1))
 (segment (start 292.1 139.7) (end 292.1 142.24) (width 0.508) (layer B.Cu) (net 1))
 (segment (start 292.1 142.24) (end 299.72 142.24) (width 0.508) (layer B.Cu) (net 1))
 (segment (start 299.72 140.798076) (end 300.76 139.758076) (width 0.508) (layer B.Cu) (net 1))
 (segment (start 299.72 142.24) (end 299.72 140.798076) (width 0.508) (layer B.Cu) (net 1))
 (segment (start 269.24 134.62) (end 269.24 137.16) (width 0.508) (layer B.Cu) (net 1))
 (via (at 269.24 137.16) (size 0.889) (drill 0.635) (layers F.Cu B.Cu) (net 1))
 (segment (start 269.24 137.16) (end 271.78 139.7) (width 0.508) (layer F.Cu) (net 1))
 (segment (start 271.78 139.7) (end 274.32 139.7) (width 0.508) (layer F.Cu) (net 1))
 (segment (start 261.62 114.3) (end 261.62 119.38) (width 0.508) (layer B.Cu) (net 32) (status 30))
 (segment (start 259.08 114.3) (end 259.08 119.38) (width 0.508) (layer B.Cu) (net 33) (status 30))
 (segment (start 256.54 119.38) (end 256.54 114.3) (width 0.508) (layer B.Cu) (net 34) (status 30))
 (segment (start 254 114.3) (end 254 119.38) (width 0.508) (layer B.Cu) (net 35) (status 30))
 (segment (start 271.78 114.3) (end 271.78 115.49) (width 0.508) (layer B.Cu) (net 44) (status 30))
 (segment (start 304.8 133.521924) (end 303.76 134.561924) (width 0.508) (layer B.Cu) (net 2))
 (segment (start 304.8 129.54) (end 304.8 133.521924) (width 0.508) (layer B.Cu) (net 2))
 (segment (start 302.26 125.81) (end 302.26 129.54) (width 0.508) (layer B.Cu) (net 45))
 (segment (start 291.465 135.89) (end 289.687 135.89) (width 0.508) (layer B.Cu) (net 4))
 (segment (start 289.687 135.89) (end 287.082601 138.494399) (width 0.508) (layer B.Cu) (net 4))
 (segment (start 283.845 135.89) (end 283.845 138.494399) (width 0.508) (layer B.Cu) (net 6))
 (segment (start 243.84 134.62) (end 243.84 138.494399) (width 0.508) (layer B.Cu) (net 17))
 (segment (start 246.38 134.62) (end 246.38 138.494399) (width 0.508) (layer B.Cu) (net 18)))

